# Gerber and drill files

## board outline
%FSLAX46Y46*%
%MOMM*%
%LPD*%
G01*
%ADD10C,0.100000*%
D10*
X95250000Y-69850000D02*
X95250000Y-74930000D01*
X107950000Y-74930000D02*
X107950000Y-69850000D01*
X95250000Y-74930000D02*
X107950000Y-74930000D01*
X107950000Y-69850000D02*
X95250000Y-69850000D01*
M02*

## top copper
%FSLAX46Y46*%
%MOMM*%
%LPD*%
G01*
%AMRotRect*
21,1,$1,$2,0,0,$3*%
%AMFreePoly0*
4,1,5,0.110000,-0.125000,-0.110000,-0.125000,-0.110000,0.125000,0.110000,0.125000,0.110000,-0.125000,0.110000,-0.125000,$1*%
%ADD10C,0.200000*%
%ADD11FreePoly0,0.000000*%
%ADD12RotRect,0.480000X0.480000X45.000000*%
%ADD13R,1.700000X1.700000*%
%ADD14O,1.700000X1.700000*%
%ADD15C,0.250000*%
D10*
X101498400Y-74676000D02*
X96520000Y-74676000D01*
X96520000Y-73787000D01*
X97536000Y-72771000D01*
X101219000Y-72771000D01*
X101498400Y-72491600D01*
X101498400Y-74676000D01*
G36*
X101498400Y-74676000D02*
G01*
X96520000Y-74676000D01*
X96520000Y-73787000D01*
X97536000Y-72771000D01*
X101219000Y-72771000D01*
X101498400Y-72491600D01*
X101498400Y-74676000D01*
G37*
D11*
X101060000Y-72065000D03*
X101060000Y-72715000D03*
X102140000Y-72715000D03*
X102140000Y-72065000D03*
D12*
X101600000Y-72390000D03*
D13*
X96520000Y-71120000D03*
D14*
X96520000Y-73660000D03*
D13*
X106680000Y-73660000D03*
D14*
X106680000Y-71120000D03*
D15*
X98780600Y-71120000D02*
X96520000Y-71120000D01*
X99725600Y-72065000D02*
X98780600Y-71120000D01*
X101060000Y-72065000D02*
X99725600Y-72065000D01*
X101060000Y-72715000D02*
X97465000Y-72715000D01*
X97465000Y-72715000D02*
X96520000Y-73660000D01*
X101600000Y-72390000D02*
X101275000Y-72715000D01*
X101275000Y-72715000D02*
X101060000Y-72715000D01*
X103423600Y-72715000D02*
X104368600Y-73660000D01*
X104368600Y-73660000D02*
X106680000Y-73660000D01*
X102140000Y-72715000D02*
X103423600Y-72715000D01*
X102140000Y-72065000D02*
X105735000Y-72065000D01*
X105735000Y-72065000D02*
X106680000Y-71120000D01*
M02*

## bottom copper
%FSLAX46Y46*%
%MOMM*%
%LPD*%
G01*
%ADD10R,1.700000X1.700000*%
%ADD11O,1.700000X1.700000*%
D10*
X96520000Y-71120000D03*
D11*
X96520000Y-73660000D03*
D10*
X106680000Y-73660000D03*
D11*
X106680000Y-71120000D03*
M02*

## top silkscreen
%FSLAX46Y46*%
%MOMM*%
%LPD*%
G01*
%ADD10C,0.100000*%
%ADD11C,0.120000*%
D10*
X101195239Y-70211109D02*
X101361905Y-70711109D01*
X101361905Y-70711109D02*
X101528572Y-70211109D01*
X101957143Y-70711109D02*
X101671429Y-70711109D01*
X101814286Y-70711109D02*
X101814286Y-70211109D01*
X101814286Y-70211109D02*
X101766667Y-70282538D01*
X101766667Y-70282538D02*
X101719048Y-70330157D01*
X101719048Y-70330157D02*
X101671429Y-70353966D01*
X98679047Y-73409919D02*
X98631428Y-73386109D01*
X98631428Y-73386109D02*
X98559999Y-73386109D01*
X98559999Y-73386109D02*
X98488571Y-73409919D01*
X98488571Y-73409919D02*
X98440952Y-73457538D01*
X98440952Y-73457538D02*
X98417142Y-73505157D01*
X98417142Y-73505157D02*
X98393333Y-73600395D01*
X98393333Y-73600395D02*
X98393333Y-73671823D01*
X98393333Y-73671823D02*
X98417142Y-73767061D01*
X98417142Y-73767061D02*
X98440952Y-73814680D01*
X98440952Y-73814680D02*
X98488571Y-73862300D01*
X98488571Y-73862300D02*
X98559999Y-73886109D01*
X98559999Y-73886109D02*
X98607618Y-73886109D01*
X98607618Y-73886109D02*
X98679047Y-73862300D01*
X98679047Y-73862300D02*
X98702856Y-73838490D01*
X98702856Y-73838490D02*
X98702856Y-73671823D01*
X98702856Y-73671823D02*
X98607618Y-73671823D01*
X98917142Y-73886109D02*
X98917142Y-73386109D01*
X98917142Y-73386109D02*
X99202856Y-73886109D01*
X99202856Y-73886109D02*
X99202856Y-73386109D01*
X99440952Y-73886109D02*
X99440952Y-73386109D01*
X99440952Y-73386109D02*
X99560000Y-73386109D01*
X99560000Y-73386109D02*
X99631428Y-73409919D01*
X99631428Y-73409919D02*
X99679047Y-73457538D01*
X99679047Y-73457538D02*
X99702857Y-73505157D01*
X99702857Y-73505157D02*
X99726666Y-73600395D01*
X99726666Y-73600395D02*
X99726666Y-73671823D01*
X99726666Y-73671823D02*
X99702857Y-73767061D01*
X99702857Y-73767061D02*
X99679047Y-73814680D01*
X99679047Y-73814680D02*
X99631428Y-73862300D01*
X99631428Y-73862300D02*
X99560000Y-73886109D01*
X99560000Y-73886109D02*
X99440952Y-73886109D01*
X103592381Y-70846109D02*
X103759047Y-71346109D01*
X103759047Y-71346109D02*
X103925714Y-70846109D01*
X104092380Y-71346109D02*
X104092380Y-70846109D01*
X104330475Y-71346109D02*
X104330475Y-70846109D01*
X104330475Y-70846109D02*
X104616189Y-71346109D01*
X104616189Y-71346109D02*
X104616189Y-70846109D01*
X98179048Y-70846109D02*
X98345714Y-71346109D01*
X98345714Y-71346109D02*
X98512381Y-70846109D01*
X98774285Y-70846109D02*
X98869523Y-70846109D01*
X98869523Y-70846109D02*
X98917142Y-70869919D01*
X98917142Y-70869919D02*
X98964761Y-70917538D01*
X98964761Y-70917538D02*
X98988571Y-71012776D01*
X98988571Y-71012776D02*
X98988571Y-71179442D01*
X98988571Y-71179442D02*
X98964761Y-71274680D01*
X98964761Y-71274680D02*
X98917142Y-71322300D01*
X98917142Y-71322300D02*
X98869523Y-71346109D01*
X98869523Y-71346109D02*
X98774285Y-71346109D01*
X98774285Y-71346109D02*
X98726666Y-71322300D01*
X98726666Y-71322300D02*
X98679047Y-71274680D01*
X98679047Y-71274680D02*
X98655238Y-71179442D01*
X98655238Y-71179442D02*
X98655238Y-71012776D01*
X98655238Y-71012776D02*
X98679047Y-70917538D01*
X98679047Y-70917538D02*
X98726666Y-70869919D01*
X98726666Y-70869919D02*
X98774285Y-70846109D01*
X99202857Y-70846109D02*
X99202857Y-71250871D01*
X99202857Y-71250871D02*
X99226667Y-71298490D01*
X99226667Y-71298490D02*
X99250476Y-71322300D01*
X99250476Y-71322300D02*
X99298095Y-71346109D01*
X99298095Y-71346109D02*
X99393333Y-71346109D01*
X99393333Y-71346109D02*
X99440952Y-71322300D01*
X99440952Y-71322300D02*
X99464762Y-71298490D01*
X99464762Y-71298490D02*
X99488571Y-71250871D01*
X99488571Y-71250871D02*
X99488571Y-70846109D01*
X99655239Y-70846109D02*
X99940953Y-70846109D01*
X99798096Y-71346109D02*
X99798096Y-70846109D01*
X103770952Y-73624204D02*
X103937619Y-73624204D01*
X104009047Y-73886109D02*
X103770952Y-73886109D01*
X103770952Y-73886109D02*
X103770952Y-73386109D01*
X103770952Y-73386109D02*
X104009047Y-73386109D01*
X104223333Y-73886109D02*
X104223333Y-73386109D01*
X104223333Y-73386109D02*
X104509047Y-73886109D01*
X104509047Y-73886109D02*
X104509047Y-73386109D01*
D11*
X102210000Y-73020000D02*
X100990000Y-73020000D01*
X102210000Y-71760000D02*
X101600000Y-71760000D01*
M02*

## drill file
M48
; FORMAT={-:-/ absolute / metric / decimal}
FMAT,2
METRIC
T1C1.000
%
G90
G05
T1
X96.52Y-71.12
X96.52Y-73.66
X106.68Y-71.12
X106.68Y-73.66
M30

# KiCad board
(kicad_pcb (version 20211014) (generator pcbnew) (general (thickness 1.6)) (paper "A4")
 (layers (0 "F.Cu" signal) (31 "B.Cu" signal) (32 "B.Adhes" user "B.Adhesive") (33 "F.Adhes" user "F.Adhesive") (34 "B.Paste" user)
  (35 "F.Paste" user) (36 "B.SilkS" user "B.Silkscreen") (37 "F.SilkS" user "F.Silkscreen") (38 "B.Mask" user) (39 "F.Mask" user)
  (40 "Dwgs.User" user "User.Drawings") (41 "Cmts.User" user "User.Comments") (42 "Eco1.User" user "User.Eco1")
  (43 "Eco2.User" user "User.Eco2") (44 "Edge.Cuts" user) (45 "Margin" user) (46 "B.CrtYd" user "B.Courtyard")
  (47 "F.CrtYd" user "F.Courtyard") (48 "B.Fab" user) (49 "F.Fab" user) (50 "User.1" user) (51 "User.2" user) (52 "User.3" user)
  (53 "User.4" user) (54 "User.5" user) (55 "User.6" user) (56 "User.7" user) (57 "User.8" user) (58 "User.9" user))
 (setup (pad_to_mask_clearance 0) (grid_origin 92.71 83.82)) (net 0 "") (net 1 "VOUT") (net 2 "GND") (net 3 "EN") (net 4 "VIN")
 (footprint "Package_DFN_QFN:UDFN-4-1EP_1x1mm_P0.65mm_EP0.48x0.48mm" (layer "F.Cu") (at 101.6 72.39)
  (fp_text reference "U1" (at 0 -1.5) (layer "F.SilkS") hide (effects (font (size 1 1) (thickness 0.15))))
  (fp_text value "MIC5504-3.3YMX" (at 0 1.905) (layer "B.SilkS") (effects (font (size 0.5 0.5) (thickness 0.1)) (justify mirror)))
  (fp_line (start 0.61 0.63) (end -0.61 0.63) (layer "F.SilkS") (width 0.12))
  (fp_line (start 0.61 -0.63) (end 0 -0.63) (layer "F.SilkS") (width 0.12))
  (pad "1" smd custom (at -0.54 -0.325) (size 0.22 0.25) (layers "F.Cu" "F.Paste" "F.Mask") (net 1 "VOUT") (zone_connect 2)
   (options (clearance outline) (anchor rect)) (primitives))
  (pad "2" smd custom (at -0.54 0.325) (size 0.22 0.25) (layers "F.Cu" "F.Paste" "F.Mask") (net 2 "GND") (zone_connect 2)
   (options (clearance outline) (anchor rect)) (primitives))
  (pad "3" smd custom (at 0.54 0.325) (size 0.22 0.25) (layers "F.Cu" "F.Paste" "F.Mask") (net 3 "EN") (zone_connect 2)
   (options (clearance outline) (anchor rect)) (primitives))
  (pad "4" smd custom (at 0.54 -0.325) (size 0.22 0.25) (layers "F.Cu" "F.Paste" "F.Mask") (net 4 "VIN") (zone_connect 2)
   (options (clearance outline) (anchor rect)) (primitives))
  (pad "5" smd rect (at 0 0 45) (size 0.48 0.48) (layers "F.Cu" "F.Paste" "F.Mask") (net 2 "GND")))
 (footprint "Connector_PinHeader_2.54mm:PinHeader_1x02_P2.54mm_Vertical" (layer "B.Cu") (at 96.52 71.12 180)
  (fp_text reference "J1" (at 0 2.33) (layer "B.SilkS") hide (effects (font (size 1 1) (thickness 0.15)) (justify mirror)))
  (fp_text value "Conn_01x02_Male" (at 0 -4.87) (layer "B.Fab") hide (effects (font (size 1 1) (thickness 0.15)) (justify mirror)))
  (pad "1" thru_hole rect (at 0 0 180) (size 1.7 1.7) (drill 1) (layers *.Cu *.Mask) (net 1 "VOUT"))
  (pad "2" thru_hole oval (at 0 -2.54 180) (size 1.7 1.7) (drill 1) (layers *.Cu *.Mask) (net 2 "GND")))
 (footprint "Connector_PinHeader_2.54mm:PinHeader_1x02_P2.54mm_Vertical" (layer "B.Cu") (at 106.68 73.66)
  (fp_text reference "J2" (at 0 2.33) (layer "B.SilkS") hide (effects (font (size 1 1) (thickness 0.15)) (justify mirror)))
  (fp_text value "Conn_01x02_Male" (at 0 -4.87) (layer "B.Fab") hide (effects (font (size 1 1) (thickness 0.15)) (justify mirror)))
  (pad "1" thru_hole rect (at 0 0) (size 1.7 1.7) (drill 1) (layers *.Cu *.Mask) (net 3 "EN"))
  (pad "2" thru_hole oval (at 0 -2.54) (size 1.7 1.7) (drill 1) (layers *.Cu *.Mask) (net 4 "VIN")))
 (gr_poly
  (pts (xy 101.4984 74.676) (xy 96.52 74.676) (xy 96.52 73.787) (xy 97.536 72.771) (xy 101.219 72.771) (xy 101.4984 72.4916)) (layer "F.Cu")
  (width 0.2) (fill solid))
 (gr_line (start 95.25 69.85) (end 95.25 74.93) (layer "Edge.Cuts") (width 0.1))
 (gr_line (start 107.95 74.93) (end 107.95 69.85) (layer "Edge.Cuts") (width 0.1))
 (gr_line (start 95.25 74.93) (end 107.95 74.93) (layer "Edge.Cuts") (width 0.1))
 (gr_line (start 107.95 69.85) (end 95.25 69.85) (layer "Edge.Cuts") (width 0.1))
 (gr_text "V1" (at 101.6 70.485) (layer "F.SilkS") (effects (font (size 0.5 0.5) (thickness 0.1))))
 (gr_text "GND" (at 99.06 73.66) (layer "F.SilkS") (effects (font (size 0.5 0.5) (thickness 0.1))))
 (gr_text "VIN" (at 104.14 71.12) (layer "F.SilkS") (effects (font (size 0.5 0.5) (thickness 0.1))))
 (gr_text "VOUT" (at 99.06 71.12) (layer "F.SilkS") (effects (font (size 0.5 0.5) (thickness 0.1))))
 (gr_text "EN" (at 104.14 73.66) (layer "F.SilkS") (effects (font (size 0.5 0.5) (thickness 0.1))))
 (segment (start 98.7806 71.12) (end 96.52 71.12) (width 0.25) (layer "F.Cu") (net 1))
 (segment (start 99.7256 72.065) (end 98.7806 71.12) (width 0.25) (layer "F.Cu") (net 1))
 (segment (start 101.06 72.065) (end 99.7256 72.065) (width 0.25) (layer "F.Cu") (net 1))
 (segment (start 101.06 72.715) (end 97.465 72.715) (width 0.25) (layer "F.Cu") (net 2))
 (segment (start 97.465 72.715) (end 96.52 73.66) (width 0.25) (layer "F.Cu") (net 2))
 (segment (start 101.6 72.39) (end 101.275 72.715) (width 0.25) (layer "F.Cu") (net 2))
 (segment (start 101.275 72.715) (end 101.06 72.715) (width 0.25) (layer "F.Cu") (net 2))
 (segment (start 103.4236 72.715) (end 104.3686 73.66) (width 0.25) (layer "F.Cu") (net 3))
 (segment (start 104.3686 73.66) (end 106.68 73.66) (width 0.25) (layer "F.Cu") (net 3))
 (segment (start 102.14 72.715) (end 103.4236 72.715) (width 0.25) (layer "F.Cu") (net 3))
 (segment (start 102.14 72.065) (end 105.735 72.065) (width 0.25) (layer "F.Cu") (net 4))
 (segment (start 105.735 72.065) (end 106.68 71.12) (width 0.25) (layer "F.Cu") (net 4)))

